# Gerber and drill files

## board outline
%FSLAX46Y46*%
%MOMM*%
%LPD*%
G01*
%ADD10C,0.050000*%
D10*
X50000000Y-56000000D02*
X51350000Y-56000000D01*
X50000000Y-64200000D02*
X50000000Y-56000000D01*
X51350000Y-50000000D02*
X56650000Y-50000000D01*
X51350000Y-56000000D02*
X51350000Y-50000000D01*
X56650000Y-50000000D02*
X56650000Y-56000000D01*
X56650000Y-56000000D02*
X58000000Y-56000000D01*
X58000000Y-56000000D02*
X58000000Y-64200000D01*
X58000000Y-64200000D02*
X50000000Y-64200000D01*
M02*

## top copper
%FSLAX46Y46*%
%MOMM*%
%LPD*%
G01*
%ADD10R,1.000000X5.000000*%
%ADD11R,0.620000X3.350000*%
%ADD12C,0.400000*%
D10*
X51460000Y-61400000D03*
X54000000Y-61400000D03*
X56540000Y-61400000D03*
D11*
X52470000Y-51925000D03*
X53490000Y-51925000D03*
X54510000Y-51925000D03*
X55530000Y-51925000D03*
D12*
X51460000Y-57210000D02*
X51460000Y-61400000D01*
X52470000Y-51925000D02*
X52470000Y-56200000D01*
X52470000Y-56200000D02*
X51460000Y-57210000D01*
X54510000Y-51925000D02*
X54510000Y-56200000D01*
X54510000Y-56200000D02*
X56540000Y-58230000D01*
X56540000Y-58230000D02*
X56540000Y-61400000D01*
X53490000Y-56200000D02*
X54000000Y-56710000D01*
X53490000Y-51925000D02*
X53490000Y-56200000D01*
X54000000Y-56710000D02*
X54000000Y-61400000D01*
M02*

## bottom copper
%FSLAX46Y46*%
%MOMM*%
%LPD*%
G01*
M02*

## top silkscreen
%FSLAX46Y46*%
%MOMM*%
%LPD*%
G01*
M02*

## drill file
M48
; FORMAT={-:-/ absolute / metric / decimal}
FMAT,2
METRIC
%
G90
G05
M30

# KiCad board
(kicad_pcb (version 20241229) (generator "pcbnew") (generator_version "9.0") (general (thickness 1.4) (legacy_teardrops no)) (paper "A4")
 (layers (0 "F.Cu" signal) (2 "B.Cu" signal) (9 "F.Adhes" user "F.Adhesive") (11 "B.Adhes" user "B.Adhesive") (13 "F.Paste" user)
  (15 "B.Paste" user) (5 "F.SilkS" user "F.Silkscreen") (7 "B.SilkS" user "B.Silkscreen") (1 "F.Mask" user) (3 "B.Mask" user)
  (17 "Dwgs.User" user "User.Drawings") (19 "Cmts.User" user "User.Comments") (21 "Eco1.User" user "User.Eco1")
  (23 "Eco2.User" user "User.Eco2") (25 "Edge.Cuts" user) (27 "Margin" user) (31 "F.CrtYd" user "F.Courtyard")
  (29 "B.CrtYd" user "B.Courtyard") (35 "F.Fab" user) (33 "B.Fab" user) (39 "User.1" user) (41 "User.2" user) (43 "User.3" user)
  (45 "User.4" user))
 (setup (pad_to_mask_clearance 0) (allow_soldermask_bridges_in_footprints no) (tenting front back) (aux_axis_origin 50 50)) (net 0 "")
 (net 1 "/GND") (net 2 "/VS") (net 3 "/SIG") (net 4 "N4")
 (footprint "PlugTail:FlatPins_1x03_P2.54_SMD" (layer "F.Cu") (at 54 61.4)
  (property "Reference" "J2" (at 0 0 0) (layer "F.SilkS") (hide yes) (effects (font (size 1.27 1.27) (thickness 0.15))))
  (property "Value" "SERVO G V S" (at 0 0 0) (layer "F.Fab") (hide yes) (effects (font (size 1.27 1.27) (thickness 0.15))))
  (pad "1" smd rect (at -2.54 0) (size 1 5) (layers "F.Cu" "F.Mask") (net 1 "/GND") (thermal_bridge_angle 45))
  (pad "2" smd rect (at 0 0) (size 1 5) (layers "F.Cu" "F.Mask") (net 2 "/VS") (thermal_bridge_angle 45))
  (pad "3" smd rect (at 2.54 0) (size 1 5) (layers "F.Cu" "F.Mask") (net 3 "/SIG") (thermal_bridge_angle 45)))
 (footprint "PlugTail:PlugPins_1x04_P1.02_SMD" (layer "F.Cu") (at 54 50)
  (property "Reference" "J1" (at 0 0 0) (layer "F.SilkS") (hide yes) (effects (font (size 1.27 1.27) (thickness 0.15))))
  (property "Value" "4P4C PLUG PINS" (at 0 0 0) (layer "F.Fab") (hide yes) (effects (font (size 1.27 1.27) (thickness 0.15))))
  (pad "1" smd rect (at -1.53 1.925) (size 0.62 3.35) (layers "F.Cu" "F.Mask") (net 1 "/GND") (thermal_bridge_angle 45))
  (pad "2" smd rect (at -0.51 1.925) (size 0.62 3.35) (layers "F.Cu" "F.Mask") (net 2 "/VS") (thermal_bridge_angle 45))
  (pad "3" smd rect (at 0.51 1.925) (size 0.62 3.35) (layers "F.Cu" "F.Mask") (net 3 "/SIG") (thermal_bridge_angle 45))
  (pad "4" smd rect (at 1.53 1.925) (size 0.62 3.35) (layers "F.Cu" "F.Mask") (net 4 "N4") (thermal_bridge_angle 45)))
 (gr_line (start 50 56) (end 51.35 56) (stroke (width 0.05) (type default)) (layer "Edge.Cuts"))
 (gr_line (start 50 64.2) (end 50 56) (stroke (width 0.05) (type default)) (layer "Edge.Cuts"))
 (gr_line (start 51.35 50) (end 56.65 50) (stroke (width 0.05) (type default)) (layer "Edge.Cuts"))
 (gr_line (start 51.35 56) (end 51.35 50) (stroke (width 0.05) (type default)) (layer "Edge.Cuts"))
 (gr_line (start 56.65 50) (end 56.65 56) (stroke (width 0.05) (type default)) (layer "Edge.Cuts"))
 (gr_line (start 56.65 56) (end 58 56) (stroke (width 0.05) (type default)) (layer "Edge.Cuts"))
 (gr_line (start 58 56) (end 58 64.2) (stroke (width 0.05) (type default)) (layer "Edge.Cuts"))
 (gr_line (start 58 64.2) (end 50 64.2) (stroke (width 0.05) (type default)) (layer "Edge.Cuts"))
 (segment (start 51.46 57.21) (end 51.46 61.4) (width 0.4) (layer "F.Cu") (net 1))
 (segment (start 52.47 51.925) (end 52.47 56.2) (width 0.4) (layer "F.Cu") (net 1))
 (segment (start 52.47 56.2) (end 51.46 57.21) (width 0.4) (layer "F.Cu") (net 1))
 (segment (start 54.51 51.925) (end 54.51 56.2) (width 0.4) (layer "F.Cu") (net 3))
 (segment (start 54.51 56.2) (end 56.54 58.23) (width 0.4) (layer "F.Cu") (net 3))
 (segment (start 56.54 58.23) (end 56.54 61.4) (width 0.4) (layer "F.Cu") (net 3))
 (segment (start 53.49 56.2) (end 54 56.71) (width 0.4) (layer "F.Cu") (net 2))
 (segment (start 53.49 51.925) (end 53.49 56.2) (width 0.4) (layer "F.Cu") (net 2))
 (segment (start 54 56.71) (end 54 61.4) (width 0.4) (layer "F.Cu") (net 2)))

